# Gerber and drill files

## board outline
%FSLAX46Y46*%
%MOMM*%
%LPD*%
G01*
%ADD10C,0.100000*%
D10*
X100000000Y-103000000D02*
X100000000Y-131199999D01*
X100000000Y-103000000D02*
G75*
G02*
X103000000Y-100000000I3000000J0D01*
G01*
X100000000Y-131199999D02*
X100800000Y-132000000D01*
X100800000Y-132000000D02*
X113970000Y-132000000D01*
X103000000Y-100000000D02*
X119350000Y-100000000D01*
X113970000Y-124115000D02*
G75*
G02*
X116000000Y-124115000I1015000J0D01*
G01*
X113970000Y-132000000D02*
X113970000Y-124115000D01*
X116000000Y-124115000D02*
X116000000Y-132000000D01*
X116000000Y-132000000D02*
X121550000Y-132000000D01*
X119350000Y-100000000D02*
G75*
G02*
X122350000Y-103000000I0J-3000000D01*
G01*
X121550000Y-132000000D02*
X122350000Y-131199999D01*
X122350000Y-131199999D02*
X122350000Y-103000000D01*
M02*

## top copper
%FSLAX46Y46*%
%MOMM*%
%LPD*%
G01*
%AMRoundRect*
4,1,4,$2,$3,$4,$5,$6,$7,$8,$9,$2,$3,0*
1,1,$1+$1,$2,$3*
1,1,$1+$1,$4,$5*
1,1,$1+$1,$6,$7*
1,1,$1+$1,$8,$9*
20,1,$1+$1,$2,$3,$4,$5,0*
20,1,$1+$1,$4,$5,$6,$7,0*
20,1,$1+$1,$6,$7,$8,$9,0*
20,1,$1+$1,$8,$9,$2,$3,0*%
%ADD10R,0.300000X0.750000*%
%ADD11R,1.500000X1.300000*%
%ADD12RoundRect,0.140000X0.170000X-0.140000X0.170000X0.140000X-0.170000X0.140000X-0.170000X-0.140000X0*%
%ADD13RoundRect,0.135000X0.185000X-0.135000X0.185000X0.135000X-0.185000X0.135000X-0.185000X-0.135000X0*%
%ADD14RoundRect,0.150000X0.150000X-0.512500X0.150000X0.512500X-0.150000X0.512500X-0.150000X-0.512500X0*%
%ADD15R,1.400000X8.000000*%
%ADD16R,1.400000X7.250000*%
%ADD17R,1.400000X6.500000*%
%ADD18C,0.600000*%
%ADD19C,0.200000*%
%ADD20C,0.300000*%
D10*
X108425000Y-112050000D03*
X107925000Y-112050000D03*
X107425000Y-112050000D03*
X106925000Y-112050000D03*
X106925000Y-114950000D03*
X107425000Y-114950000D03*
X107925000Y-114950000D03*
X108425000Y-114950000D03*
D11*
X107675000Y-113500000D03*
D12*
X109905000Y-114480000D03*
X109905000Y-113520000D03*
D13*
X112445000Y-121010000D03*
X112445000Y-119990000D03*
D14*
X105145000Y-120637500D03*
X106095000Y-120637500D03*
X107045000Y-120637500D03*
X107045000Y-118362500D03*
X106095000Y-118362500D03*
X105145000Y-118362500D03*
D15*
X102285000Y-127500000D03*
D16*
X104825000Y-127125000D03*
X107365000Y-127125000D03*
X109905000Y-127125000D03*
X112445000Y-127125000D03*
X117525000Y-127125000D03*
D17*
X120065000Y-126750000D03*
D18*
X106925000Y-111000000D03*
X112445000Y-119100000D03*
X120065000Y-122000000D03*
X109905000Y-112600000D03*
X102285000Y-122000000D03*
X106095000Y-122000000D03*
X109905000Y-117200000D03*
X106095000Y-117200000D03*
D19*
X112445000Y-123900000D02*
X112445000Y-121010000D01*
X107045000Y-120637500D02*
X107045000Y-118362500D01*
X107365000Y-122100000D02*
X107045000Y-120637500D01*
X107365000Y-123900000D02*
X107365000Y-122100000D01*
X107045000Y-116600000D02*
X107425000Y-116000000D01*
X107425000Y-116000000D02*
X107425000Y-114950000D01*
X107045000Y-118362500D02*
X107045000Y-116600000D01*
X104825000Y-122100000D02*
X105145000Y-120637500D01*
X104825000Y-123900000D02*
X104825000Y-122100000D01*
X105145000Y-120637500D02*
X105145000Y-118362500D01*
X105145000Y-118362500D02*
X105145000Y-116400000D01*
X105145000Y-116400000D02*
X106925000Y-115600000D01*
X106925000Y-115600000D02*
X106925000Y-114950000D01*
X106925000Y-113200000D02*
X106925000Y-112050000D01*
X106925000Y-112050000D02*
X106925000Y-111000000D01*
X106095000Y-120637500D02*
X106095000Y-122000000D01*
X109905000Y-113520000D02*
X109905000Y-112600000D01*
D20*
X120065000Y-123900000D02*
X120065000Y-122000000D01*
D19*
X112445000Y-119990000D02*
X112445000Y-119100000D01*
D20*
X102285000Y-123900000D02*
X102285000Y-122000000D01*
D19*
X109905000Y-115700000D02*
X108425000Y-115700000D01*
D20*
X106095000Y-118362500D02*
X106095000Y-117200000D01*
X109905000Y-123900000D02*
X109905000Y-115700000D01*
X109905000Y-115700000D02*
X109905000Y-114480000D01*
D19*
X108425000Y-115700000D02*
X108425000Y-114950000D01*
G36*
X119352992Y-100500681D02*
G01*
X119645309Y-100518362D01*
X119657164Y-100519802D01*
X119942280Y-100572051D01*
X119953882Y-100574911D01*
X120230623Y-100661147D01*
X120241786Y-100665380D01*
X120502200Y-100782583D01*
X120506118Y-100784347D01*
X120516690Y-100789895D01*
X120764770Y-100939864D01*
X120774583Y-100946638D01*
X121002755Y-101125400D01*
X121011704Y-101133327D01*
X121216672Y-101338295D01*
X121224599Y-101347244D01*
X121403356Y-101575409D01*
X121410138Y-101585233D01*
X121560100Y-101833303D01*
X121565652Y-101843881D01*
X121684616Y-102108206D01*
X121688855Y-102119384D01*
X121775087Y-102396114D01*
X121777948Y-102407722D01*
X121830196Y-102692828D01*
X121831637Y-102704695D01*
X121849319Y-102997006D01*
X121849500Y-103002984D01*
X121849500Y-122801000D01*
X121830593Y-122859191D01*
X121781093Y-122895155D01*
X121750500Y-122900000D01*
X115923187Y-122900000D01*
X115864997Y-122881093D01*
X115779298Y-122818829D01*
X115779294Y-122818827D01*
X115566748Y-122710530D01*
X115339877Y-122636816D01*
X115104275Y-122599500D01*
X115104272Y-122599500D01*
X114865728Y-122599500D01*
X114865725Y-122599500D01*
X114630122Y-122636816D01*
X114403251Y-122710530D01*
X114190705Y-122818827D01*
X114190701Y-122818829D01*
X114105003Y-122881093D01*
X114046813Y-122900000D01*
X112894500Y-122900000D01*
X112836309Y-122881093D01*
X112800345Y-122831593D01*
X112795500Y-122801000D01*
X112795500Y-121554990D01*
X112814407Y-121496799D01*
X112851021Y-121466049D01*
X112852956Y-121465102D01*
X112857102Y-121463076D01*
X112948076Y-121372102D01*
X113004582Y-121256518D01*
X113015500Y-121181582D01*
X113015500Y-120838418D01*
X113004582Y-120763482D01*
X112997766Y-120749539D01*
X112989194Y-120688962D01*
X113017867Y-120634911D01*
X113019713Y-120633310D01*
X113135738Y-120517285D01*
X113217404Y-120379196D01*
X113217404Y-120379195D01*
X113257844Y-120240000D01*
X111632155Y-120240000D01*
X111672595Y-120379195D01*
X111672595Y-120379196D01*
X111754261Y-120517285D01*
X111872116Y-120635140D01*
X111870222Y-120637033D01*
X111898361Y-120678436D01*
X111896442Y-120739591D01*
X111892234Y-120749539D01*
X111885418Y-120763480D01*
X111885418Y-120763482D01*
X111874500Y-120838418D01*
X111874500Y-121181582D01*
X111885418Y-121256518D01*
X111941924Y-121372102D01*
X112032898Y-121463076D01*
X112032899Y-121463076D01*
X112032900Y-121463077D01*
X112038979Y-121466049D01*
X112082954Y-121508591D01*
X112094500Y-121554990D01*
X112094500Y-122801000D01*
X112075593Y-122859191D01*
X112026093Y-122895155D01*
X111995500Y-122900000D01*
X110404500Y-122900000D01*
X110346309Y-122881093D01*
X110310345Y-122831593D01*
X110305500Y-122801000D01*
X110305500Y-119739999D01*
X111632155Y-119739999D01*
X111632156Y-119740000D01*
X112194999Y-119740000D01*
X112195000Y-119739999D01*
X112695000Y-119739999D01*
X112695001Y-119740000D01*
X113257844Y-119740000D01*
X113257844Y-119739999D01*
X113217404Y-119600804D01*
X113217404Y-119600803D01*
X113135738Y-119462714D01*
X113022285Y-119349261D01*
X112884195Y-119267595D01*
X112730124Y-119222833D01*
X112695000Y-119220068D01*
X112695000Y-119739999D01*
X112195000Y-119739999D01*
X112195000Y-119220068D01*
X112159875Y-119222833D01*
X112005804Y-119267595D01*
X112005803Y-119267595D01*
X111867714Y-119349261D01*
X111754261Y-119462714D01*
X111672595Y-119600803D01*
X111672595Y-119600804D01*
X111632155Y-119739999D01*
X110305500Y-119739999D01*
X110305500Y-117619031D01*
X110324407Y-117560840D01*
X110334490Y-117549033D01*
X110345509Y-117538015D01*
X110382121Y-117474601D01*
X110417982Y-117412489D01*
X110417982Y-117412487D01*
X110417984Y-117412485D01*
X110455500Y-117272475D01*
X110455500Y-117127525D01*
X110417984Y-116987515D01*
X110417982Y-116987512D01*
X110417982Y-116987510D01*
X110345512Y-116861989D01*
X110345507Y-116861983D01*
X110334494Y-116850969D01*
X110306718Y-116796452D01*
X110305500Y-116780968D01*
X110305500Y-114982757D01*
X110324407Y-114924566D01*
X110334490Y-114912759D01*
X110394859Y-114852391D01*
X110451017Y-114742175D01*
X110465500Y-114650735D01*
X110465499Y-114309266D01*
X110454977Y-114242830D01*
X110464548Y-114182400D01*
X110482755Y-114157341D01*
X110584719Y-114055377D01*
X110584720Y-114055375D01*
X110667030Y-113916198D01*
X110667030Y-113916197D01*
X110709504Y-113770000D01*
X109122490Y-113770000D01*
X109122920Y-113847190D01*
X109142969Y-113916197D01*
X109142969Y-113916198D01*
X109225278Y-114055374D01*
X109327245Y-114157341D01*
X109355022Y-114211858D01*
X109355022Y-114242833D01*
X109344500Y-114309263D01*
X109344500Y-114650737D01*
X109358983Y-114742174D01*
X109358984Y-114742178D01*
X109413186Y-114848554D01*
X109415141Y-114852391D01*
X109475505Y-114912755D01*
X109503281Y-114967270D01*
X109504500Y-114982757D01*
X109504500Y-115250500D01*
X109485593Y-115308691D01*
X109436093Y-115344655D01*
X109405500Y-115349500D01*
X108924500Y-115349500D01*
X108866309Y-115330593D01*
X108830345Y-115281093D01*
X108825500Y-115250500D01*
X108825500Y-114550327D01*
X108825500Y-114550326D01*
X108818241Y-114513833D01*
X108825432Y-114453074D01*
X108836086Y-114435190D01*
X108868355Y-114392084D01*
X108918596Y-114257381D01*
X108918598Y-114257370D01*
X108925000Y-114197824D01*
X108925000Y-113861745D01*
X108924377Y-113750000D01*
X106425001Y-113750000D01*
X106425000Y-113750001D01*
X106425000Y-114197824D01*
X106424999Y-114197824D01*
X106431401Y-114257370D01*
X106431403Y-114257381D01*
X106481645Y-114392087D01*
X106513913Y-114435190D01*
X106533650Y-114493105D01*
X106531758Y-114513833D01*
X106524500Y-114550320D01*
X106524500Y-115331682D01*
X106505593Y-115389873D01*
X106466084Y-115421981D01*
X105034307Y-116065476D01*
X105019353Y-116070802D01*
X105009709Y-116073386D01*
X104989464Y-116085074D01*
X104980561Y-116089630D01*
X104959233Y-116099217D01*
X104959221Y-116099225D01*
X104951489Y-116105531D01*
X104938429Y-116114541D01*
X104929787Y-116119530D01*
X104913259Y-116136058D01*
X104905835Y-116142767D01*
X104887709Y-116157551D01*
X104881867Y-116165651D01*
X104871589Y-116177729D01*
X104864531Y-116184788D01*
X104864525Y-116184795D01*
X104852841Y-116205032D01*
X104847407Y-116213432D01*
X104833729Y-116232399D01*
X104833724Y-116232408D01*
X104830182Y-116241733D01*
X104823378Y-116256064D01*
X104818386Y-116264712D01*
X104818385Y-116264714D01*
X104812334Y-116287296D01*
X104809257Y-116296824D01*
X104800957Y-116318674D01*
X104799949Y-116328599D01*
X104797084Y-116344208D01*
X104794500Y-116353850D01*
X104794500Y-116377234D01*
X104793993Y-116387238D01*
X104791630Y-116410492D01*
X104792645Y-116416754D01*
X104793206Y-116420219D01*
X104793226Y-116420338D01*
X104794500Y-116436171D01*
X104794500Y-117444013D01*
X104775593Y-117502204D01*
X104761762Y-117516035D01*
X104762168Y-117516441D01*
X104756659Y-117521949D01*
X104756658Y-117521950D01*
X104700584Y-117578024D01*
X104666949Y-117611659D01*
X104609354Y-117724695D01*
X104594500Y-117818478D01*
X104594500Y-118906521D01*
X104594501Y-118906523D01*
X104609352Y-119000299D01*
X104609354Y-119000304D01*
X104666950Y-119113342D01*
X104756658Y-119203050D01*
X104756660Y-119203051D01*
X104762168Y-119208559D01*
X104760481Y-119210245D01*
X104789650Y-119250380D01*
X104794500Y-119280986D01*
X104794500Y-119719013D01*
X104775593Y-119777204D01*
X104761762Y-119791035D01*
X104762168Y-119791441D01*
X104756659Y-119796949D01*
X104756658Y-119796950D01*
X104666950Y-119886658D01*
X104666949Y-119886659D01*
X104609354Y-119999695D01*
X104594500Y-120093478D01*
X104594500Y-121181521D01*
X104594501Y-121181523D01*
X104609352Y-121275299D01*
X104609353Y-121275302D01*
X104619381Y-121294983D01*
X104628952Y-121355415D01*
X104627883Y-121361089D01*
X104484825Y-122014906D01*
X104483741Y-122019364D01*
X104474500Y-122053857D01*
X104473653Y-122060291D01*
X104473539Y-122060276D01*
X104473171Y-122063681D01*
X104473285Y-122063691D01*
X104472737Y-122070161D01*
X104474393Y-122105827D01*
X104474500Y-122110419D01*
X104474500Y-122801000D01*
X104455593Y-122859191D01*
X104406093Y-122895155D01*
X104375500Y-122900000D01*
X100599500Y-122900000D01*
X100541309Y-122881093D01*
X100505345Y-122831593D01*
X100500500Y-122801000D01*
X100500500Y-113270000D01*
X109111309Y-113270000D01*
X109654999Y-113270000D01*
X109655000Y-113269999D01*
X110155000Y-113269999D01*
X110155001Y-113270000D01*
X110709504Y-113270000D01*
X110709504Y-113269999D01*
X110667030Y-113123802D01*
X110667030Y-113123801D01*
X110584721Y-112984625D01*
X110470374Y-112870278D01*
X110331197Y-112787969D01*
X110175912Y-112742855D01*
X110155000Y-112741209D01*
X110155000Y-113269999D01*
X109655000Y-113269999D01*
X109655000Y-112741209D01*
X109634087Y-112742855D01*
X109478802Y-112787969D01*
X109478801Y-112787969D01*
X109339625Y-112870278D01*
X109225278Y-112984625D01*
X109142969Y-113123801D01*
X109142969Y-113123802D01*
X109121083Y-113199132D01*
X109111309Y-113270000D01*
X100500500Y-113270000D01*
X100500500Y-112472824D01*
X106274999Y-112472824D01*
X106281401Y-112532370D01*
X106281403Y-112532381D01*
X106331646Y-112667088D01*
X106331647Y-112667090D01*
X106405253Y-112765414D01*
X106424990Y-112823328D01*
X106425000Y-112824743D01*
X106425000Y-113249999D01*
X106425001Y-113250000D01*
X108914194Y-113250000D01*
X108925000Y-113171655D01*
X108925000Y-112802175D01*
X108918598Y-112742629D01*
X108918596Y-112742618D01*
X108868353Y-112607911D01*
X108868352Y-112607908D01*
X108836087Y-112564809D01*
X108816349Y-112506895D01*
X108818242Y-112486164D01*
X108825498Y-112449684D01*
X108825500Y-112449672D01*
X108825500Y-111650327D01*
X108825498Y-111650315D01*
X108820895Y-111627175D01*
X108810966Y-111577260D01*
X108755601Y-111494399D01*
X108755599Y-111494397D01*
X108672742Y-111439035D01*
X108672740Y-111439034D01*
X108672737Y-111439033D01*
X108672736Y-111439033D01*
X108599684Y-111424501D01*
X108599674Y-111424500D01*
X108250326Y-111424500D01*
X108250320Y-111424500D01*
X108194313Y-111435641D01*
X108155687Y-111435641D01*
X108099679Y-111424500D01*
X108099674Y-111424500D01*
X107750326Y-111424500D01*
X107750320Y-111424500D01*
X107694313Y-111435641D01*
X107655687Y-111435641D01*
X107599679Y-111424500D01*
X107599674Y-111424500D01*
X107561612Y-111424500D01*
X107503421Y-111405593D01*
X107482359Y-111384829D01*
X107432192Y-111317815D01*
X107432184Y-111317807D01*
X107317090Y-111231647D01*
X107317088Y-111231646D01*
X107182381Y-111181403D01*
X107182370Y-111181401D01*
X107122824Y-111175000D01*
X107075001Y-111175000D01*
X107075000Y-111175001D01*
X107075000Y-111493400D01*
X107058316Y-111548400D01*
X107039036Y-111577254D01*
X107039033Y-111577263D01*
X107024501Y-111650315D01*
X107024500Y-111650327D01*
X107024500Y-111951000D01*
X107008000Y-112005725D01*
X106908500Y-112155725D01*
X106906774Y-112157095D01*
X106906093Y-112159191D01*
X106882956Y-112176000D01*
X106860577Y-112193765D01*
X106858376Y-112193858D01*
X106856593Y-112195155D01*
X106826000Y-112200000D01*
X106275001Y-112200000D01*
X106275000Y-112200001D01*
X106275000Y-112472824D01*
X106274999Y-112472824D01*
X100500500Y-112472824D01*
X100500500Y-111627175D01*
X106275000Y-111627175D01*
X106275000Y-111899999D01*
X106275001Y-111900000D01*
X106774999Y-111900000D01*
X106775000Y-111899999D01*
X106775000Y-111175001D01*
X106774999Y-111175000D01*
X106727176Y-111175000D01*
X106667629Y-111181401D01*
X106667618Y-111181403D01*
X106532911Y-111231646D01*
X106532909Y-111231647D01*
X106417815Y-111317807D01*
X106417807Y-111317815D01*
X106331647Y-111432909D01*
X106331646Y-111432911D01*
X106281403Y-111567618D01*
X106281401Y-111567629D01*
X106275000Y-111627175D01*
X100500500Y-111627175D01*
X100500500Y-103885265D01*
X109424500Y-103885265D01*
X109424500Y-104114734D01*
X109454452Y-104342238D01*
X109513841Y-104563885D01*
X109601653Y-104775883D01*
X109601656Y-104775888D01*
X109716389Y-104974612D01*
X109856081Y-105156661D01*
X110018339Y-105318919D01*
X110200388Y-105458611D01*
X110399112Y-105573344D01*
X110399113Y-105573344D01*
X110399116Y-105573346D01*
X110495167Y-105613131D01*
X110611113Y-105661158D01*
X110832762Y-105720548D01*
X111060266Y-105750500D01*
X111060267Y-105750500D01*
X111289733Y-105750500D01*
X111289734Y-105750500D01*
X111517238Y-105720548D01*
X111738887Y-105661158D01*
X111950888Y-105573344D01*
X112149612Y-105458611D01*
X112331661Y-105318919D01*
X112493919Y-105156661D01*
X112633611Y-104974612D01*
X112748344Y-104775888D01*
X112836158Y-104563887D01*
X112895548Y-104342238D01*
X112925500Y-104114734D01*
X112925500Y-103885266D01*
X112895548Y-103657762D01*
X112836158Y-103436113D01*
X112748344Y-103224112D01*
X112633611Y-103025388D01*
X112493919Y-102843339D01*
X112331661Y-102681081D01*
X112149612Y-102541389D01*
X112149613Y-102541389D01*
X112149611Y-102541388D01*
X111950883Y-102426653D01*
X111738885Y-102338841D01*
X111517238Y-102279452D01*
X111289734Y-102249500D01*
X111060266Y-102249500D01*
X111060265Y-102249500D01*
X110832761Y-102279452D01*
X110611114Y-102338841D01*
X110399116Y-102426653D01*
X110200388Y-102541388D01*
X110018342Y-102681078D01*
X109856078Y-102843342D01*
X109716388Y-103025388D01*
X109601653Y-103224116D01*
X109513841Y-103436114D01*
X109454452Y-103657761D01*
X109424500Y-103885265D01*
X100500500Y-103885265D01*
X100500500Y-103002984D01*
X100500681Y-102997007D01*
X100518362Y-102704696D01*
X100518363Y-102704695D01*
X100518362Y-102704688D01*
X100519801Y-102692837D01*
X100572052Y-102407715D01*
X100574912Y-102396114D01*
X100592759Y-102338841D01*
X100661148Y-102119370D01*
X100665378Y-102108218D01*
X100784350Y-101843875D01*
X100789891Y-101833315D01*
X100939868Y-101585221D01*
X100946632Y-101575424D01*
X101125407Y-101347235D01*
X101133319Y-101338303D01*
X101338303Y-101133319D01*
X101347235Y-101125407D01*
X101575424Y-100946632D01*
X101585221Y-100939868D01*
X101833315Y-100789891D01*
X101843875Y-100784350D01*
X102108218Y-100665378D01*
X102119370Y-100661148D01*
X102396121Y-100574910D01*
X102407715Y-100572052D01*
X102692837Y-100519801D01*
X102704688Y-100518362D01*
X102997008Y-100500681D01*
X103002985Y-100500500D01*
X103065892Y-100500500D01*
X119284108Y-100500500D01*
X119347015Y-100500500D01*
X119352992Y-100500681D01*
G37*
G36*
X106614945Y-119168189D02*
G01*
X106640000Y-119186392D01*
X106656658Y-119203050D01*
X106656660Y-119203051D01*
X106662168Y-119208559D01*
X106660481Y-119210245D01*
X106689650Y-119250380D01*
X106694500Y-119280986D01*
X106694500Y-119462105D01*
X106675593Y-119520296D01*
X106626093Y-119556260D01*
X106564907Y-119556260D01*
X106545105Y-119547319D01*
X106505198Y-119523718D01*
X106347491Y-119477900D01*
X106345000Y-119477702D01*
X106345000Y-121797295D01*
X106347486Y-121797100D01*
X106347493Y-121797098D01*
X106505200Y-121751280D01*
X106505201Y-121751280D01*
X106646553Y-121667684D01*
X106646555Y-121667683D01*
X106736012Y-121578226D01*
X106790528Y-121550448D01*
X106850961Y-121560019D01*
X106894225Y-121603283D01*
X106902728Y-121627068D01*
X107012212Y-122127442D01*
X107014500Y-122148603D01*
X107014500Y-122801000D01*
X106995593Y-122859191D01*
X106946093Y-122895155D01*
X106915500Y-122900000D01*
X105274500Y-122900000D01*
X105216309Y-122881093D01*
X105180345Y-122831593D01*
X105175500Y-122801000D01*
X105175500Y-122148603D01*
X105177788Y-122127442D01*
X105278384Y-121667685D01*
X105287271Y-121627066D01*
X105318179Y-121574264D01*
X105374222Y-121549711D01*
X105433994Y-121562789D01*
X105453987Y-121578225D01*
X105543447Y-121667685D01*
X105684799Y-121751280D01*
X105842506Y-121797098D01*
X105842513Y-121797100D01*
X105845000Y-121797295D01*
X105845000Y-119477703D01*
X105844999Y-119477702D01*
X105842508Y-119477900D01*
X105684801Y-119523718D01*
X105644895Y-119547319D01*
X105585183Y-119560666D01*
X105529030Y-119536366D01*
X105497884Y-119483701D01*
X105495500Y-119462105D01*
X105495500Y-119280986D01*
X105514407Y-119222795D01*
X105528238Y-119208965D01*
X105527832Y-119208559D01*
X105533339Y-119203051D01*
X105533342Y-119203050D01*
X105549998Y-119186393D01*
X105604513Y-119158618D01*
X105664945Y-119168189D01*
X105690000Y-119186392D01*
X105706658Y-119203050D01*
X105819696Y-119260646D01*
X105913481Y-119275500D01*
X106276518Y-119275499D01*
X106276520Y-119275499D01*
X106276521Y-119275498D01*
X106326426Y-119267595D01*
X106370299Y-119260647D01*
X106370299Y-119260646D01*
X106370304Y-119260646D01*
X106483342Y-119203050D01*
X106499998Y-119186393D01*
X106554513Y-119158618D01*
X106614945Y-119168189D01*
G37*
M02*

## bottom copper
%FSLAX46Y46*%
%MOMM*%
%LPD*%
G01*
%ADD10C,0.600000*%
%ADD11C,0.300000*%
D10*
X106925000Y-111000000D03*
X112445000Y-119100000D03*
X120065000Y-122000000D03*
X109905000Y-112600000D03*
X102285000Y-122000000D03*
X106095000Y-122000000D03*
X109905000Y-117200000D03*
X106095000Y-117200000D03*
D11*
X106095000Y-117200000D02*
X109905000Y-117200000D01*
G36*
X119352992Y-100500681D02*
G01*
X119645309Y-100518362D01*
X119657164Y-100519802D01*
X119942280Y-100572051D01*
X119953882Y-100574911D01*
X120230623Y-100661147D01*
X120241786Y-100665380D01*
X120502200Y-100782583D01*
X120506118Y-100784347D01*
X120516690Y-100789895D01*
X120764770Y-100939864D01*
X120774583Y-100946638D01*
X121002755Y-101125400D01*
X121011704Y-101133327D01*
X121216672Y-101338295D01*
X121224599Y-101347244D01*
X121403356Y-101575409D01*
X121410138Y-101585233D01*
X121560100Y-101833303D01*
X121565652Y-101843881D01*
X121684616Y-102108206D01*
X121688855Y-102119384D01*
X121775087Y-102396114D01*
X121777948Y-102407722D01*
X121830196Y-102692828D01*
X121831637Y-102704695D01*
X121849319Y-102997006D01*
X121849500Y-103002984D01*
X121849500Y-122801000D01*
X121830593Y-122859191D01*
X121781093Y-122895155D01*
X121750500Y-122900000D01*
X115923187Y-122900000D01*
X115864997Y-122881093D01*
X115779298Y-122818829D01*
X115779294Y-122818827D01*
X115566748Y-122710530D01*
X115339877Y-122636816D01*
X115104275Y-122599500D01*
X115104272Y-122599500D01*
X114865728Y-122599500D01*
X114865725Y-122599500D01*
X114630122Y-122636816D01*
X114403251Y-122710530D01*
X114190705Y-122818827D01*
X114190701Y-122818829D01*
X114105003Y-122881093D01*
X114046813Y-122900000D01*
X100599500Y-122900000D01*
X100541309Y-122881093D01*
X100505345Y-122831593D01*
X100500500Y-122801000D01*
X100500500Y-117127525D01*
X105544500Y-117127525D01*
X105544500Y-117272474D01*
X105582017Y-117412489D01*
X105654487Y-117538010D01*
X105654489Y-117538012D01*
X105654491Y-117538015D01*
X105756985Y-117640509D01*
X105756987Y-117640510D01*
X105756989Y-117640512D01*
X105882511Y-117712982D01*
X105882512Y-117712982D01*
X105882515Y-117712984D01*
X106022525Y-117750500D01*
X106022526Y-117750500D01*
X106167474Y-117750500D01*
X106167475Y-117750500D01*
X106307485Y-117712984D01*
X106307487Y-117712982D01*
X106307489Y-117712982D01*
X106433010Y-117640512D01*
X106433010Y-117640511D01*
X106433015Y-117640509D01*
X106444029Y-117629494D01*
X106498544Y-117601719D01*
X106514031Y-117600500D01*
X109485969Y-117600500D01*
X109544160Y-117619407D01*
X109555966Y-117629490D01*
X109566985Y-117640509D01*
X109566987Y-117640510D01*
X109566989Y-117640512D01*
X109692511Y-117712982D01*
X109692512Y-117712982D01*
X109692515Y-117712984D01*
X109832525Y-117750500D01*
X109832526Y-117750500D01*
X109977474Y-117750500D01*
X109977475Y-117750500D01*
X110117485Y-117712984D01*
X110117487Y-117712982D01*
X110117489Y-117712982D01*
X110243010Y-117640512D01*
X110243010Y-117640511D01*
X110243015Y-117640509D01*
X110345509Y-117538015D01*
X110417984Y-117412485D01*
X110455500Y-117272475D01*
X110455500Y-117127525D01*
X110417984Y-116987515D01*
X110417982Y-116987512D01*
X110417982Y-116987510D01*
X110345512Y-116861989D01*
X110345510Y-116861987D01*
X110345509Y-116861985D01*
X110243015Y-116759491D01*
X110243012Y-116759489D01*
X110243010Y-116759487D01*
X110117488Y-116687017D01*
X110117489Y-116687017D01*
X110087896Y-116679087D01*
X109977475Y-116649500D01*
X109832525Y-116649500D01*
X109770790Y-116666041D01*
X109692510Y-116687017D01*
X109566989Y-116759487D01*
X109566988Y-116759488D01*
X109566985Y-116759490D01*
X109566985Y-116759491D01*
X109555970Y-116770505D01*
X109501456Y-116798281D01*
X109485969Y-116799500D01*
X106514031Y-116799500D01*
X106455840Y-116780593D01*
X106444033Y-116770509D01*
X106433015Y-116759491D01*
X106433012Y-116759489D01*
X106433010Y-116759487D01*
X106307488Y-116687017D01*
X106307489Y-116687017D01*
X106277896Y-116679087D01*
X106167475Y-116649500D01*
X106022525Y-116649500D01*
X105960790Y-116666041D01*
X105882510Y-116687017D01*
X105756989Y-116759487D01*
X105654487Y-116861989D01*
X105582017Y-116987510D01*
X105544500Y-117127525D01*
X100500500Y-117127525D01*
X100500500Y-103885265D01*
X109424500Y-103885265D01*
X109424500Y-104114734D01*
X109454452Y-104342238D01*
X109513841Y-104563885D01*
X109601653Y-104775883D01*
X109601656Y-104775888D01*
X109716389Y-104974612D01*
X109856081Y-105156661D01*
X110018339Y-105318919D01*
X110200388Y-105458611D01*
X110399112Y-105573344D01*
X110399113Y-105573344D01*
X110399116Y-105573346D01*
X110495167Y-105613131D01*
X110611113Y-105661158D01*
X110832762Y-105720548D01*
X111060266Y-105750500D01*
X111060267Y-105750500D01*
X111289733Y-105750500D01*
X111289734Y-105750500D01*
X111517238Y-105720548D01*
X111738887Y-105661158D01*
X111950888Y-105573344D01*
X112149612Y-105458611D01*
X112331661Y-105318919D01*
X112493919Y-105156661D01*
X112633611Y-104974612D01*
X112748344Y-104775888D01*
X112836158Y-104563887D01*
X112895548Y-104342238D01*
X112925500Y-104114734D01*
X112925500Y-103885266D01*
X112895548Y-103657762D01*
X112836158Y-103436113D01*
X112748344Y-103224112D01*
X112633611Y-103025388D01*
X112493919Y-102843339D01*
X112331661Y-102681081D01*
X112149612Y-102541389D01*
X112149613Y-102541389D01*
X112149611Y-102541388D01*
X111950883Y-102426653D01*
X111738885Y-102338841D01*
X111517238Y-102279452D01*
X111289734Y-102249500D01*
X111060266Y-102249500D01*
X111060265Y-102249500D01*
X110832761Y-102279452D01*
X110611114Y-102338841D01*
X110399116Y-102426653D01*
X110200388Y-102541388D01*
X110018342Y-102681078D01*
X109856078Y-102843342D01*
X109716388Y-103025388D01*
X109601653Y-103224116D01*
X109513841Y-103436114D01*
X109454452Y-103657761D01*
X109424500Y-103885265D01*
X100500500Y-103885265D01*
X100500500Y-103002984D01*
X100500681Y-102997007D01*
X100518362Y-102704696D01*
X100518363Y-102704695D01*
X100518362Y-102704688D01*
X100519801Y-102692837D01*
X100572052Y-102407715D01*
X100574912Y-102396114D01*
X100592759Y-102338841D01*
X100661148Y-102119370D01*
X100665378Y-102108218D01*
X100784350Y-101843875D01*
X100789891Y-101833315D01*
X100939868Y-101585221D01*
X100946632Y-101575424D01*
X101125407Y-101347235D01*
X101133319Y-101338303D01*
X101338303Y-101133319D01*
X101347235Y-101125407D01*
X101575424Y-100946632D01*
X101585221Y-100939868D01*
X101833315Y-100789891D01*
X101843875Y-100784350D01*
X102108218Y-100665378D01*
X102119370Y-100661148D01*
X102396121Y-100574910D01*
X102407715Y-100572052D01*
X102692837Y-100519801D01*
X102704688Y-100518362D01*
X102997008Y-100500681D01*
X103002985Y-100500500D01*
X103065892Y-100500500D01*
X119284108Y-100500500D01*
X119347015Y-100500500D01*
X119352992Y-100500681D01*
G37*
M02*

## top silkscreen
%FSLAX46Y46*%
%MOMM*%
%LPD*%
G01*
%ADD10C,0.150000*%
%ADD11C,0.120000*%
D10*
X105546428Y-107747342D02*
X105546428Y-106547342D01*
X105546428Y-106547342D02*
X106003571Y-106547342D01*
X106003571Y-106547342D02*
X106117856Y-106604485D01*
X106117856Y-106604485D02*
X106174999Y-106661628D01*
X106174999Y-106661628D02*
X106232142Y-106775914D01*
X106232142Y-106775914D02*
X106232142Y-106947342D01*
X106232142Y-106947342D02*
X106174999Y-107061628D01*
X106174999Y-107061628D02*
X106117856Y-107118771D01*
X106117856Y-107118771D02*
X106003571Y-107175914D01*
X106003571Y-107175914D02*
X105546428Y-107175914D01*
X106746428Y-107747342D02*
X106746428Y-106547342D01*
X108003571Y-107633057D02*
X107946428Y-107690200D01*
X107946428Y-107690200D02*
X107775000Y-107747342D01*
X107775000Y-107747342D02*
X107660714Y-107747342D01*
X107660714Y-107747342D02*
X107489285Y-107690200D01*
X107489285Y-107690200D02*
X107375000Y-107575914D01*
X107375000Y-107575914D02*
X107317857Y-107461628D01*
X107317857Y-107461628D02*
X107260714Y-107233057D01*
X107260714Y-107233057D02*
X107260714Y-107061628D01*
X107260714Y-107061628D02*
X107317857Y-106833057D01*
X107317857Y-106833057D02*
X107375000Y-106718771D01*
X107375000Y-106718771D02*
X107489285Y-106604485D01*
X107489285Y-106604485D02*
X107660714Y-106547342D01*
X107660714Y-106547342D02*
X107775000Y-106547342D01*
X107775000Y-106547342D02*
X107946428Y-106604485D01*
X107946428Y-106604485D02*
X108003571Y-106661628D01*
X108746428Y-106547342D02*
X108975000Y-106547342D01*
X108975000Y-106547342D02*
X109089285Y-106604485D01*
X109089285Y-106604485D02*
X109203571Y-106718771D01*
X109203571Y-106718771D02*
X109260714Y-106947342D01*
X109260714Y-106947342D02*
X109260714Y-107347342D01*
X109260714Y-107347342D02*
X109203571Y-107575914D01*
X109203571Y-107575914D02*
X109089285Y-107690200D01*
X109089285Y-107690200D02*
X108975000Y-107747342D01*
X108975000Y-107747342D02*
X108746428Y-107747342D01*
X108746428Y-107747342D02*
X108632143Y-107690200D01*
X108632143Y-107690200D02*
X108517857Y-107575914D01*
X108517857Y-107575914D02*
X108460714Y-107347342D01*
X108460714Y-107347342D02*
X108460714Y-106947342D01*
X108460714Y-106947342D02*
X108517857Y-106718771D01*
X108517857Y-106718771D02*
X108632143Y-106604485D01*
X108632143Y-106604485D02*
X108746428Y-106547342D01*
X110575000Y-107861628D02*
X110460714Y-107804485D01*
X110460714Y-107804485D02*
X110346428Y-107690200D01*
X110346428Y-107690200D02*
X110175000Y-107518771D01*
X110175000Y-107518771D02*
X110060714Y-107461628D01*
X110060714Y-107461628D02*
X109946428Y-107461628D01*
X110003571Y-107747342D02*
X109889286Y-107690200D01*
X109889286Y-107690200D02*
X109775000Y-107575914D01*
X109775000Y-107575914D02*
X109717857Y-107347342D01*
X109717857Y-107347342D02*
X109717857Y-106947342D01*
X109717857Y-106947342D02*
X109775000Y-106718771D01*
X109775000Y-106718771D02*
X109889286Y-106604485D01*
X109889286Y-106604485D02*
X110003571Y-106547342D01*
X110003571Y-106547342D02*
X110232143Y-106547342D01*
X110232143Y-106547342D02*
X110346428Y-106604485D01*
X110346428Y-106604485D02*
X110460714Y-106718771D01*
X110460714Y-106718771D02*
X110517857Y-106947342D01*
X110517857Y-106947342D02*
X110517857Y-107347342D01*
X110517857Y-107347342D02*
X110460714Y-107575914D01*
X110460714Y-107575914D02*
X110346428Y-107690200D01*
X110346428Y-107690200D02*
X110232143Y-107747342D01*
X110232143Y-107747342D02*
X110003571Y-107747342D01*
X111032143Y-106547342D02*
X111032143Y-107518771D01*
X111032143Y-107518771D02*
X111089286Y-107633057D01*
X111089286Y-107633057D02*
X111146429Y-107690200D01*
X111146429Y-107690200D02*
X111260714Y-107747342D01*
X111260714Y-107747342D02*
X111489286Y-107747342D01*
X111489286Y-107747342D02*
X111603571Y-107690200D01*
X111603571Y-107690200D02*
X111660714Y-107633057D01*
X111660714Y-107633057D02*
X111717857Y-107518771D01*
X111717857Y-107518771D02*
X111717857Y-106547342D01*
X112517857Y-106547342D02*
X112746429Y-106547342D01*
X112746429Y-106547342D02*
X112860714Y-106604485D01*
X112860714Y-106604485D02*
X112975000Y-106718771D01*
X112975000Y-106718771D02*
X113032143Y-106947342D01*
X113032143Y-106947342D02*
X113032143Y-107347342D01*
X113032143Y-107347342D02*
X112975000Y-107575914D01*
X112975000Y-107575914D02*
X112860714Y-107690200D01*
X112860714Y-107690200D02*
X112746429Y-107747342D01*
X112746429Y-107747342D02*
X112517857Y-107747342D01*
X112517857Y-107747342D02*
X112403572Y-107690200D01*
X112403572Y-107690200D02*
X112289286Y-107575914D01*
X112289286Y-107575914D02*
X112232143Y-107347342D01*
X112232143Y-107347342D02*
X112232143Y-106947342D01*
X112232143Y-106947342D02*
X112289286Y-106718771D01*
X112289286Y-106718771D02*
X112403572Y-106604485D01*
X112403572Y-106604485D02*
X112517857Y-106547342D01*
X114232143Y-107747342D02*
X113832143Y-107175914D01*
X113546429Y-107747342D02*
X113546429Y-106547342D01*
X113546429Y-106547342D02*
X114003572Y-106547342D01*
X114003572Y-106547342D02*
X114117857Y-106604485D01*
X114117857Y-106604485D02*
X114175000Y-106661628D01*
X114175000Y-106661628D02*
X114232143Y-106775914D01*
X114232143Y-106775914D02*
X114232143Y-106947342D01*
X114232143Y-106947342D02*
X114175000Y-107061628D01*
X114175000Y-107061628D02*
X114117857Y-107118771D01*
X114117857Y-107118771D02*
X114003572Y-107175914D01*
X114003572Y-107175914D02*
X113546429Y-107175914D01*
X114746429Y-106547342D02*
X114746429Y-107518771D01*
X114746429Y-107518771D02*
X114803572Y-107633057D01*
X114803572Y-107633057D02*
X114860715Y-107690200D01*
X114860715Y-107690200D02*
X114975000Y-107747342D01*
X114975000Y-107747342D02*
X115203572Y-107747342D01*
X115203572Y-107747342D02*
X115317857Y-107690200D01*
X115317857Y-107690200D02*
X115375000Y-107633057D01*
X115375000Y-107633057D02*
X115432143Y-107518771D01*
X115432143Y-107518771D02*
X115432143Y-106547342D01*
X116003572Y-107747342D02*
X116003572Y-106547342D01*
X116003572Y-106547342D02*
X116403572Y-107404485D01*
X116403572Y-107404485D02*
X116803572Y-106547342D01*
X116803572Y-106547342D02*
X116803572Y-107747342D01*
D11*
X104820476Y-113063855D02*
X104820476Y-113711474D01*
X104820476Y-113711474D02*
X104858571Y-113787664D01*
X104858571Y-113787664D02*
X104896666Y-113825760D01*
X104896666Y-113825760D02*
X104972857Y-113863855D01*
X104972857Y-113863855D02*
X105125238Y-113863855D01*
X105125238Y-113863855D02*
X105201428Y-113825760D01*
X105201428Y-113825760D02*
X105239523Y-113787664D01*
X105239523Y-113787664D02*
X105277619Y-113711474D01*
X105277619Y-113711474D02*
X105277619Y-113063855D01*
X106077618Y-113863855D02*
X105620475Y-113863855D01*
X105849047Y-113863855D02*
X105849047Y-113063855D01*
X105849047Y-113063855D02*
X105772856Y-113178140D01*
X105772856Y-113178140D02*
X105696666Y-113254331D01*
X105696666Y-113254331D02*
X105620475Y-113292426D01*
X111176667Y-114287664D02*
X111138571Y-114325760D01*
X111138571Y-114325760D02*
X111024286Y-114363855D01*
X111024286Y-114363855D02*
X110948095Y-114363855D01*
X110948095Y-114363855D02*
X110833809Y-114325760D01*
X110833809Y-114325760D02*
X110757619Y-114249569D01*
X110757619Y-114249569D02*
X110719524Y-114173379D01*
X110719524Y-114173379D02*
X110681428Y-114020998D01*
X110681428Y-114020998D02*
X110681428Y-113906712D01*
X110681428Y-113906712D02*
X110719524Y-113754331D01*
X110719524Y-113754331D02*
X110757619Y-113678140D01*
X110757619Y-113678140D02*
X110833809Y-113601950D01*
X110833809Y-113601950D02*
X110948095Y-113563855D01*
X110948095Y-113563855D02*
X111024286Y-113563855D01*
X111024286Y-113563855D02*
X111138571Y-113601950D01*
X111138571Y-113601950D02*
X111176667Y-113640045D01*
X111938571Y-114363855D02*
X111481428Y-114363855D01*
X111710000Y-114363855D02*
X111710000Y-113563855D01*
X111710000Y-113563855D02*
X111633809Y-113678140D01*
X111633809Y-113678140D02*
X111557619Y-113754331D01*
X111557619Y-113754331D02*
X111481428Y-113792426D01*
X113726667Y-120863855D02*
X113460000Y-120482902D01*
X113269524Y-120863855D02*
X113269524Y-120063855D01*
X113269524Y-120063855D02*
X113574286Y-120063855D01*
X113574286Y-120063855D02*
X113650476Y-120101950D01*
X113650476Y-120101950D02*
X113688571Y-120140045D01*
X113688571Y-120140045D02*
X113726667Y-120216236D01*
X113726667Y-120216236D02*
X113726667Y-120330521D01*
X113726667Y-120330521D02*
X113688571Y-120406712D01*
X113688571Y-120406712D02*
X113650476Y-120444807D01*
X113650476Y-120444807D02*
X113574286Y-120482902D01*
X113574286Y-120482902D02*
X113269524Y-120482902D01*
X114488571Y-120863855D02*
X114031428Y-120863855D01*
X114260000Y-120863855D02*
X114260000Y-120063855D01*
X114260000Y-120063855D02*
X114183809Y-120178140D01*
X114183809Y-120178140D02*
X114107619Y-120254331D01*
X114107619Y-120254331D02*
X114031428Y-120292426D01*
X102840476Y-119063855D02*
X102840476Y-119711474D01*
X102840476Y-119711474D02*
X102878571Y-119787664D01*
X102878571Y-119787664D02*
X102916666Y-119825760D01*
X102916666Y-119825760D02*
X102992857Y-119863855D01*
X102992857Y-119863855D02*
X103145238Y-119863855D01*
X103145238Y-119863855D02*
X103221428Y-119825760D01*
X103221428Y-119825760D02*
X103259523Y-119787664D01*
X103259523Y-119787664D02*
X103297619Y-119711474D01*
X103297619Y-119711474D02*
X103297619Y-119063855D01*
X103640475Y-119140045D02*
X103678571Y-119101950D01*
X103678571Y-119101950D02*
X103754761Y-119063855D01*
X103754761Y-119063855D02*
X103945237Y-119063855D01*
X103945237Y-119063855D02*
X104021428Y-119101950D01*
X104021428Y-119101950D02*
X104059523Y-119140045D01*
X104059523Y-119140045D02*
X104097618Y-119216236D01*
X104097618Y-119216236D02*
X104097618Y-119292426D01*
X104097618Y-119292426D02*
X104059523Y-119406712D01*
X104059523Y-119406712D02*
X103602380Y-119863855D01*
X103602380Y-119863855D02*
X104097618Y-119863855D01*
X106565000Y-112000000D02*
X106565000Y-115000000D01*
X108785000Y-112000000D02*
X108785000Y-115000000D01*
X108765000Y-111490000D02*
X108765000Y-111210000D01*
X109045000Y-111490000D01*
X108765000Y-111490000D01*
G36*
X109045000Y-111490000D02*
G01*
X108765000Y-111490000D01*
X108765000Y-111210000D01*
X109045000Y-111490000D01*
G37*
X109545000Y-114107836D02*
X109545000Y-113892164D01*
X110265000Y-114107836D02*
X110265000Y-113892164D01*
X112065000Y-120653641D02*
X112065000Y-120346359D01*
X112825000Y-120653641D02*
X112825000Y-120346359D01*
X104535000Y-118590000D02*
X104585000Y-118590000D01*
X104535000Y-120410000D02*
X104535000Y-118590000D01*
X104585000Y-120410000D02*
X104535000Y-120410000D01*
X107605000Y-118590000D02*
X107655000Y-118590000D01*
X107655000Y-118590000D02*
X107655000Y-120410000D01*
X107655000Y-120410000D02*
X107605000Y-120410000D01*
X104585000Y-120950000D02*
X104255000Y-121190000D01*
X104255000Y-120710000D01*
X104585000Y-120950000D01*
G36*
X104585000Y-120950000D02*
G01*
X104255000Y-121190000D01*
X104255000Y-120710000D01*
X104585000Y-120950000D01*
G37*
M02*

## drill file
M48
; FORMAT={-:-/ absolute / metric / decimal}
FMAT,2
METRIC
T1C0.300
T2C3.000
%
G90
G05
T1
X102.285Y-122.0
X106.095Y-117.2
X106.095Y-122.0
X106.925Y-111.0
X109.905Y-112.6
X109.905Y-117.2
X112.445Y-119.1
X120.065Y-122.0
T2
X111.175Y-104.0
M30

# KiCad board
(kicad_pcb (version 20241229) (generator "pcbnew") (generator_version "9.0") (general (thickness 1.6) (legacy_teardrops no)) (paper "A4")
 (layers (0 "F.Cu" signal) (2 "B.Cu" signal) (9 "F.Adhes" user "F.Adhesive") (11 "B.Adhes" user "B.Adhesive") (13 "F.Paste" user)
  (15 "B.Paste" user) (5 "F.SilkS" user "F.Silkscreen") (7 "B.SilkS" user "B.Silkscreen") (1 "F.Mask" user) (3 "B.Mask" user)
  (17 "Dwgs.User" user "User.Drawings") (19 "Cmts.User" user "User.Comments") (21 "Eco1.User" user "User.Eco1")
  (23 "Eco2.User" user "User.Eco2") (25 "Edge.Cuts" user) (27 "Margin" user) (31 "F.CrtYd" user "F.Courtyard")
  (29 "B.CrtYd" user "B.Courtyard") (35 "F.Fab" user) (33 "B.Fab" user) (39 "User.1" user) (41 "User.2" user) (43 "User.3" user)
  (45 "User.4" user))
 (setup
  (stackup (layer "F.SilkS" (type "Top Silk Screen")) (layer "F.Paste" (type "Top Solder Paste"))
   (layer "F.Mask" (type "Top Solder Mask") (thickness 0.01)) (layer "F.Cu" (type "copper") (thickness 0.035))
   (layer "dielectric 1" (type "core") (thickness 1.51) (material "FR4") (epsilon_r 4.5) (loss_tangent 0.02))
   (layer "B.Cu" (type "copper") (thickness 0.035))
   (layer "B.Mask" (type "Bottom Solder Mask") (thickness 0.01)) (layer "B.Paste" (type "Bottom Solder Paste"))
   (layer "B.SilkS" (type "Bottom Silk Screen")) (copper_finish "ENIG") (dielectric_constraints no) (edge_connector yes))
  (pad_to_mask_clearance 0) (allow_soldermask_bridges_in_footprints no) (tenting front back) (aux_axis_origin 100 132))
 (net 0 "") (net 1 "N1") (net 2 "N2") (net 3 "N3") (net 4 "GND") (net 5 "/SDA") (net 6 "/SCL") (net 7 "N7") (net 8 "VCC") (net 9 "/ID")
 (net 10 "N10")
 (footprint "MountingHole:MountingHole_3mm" (layer "F.Cu") (at 111.175 104)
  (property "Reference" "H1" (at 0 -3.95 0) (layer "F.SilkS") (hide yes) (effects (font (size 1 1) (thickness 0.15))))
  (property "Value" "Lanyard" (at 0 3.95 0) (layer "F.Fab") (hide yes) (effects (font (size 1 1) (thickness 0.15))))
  (pad "" np_thru_hole circle (at 0 0) (size 3 3) (drill 3) (layers "*.Cu" "*.Mask")))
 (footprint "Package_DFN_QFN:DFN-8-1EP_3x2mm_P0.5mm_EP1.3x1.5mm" (layer "F.Cu") (at 107.675 113.5 -90)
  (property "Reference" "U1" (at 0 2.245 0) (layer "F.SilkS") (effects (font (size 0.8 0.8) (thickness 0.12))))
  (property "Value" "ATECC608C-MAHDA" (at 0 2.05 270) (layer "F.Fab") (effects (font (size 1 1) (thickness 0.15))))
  (fp_line (start -1.5 1.11) (end 1.5 1.11) (stroke (width 0.12) (type solid)) (layer "F.SilkS"))
  (fp_line (start -1.5 -1.11) (end 1.5 -1.11) (stroke (width 0.12) (type solid)) (layer "F.SilkS"))
  (fp_poly
   (pts (xy -2.01 -1.09) (xy -2.29 -1.09) (xy -2.01 -1.37) (xy -2.01 -1.09)) (stroke (width 0.12) (type solid)) (fill yes) (layer "F.SilkS"))
  (pad "" smd rect (at -0.325 -0.375 270) (size 0.5 0.6) (layers "F.Paste"))
  (pad "" smd rect (at -0.325 0.375 270) (size 0.5 0.6) (layers "F.Paste"))
  (pad "" smd rect (at 0.325 -0.375 270) (size 0.5 0.6) (layers "F.Paste"))
  (pad "" smd rect (at 0.325 0.375 270) (size 0.5 0.6) (layers "F.Paste"))
  (pad "1" smd rect (at -1.45 -0.75 270) (size 0.75 0.3) (layers "F.Cu" "F.Mask" "F.Paste") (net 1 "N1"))
  (pad "2" smd rect (at -1.45 -0.25 270) (size 0.75 0.3) (layers "F.Cu" "F.Mask" "F.Paste") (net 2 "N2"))
  (pad "3" smd rect (at -1.45 0.25 270) (size 0.75 0.3) (layers "F.Cu" "F.Mask" "F.Paste") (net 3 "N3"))
  (pad "4" smd rect (at -1.45 0.75 270) (size 0.75 0.3) (layers "F.Cu" "F.Mask" "F.Paste") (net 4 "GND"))
  (pad "5" smd rect (at 1.45 0.75 270) (size 0.75 0.3) (layers "F.Cu" "F.Mask" "F.Paste") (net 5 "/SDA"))
  (pad "6" smd rect (at 1.45 0.25 270) (size 0.75 0.3) (layers "F.Cu" "F.Mask" "F.Paste") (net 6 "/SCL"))
  (pad "7" smd rect (at 1.45 -0.25 270) (size 0.75 0.3) (layers "F.Cu" "F.Mask" "F.Paste") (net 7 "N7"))
  (pad "8" smd rect (at 1.45 -0.75 270) (size 0.75 0.3) (layers "F.Cu" "F.Mask" "F.Paste") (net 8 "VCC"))
  (pad "9" smd rect (at 0 0 270) (size 1.3 1.5) (layers "F.Cu" "F.Mask") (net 4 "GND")))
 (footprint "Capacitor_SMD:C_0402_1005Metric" (layer "F.Cu") (at 109.905 114 90)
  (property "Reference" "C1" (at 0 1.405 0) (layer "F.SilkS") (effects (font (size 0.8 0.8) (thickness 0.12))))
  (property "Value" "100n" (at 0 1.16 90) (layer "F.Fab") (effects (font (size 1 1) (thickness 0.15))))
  (fp_line (start -0.107836 -0.36) (end 0.107836 -0.36) (stroke (width 0.12) (type solid)) (layer "F.SilkS"))
  (fp_line (start -0.107836 0.36) (end 0.107836 0.36) (stroke (width 0.12) (type solid)) (layer "F.SilkS"))
  (pad "1" smd roundrect (at -0.48 0 90) (size 0.56 0.62) (layers "F.Cu" "F.Mask" "F.Paste") (roundrect_rratio 0.25) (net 8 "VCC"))
  (pad "2" smd roundrect (at 0.48 0 90) (size 0.56 0.62) (layers "F.Cu" "F.Mask" "F.Paste") (roundrect_rratio 0.25) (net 4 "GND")))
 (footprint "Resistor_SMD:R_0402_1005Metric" (layer "F.Cu") (at 112.445 120.5 90)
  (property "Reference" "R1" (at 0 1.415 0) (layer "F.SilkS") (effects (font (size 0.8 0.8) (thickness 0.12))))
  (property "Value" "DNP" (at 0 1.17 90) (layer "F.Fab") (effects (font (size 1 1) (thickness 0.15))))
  (fp_line (start -0.153641 -0.38) (end 0.153641 -0.38) (stroke (width 0.12) (type solid)) (layer "F.SilkS"))
  (fp_line (start -0.153641 0.38) (end 0.153641 0.38) (stroke (width 0.12) (type solid)) (layer "F.SilkS"))
  (pad "1" smd roundrect (at -0.51 0 90) (size 0.54 0.64) (layers "F.Cu" "F.Mask" "F.Paste") (roundrect_rratio 0.25) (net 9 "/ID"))
  (pad "2" smd roundrect (at 0.51 0 90) (size 0.54 0.64) (layers "F.Cu" "F.Mask" "F.Paste") (roundrect_rratio 0.25) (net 4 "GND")))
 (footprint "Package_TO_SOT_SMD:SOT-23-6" (layer "F.Cu") (at 106.095 119.5 90)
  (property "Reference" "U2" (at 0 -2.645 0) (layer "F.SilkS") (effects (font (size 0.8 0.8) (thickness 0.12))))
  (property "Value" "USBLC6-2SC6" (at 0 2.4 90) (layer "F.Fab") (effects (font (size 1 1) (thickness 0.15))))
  (fp_line (start 0.91 -1.56) (end 0.91 -1.51) (stroke (width 0.12) (type solid)) (layer "F.SilkS"))
  (fp_line (start -0.91 -1.56) (end 0.91 -1.56) (stroke (width 0.12) (type solid)) (layer "F.SilkS"))
  (fp_line (start -0.91 -1.51) (end -0.91 -1.56) (stroke (width 0.12) (type solid)) (layer "F.SilkS"))
  (fp_line (start 0.91 1.51) (end 0.91 1.56) (stroke (width 0.12) (type solid)) (layer "F.SilkS"))
  (fp_line (start 0.91 1.56) (end -0.91 1.56) (stroke (width 0.12) (type solid)) (layer "F.SilkS"))
  (fp_line (start -0.91 1.56) (end -0.91 1.51) (stroke (width 0.12) (type solid)) (layer "F.SilkS"))
  (fp_poly (pts (xy -1.45 -1.51) (xy -1.69 -1.84) (xy -1.21 -1.84)) (stroke (width 0.12) (type solid)) (fill yes) (layer "F.SilkS"))
  (pad "1" smd roundrect (at -1.1375 -0.95 90) (size 1.325 0.6) (layers "F.Cu" "F.Mask" "F.Paste") (roundrect_rratio 0.25) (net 5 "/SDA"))
  (pad "2" smd roundrect (at -1.1375 0 90) (size 1.325 0.6) (layers "F.Cu" "F.Mask" "F.Paste") (roundrect_rratio 0.25) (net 4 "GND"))
  (pad "3" smd roundrect (at -1.1375 0.95 90) (size 1.325 0.6) (layers "F.Cu" "F.Mask" "F.Paste") (roundrect_rratio 0.25) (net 6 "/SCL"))
  (pad "4" smd roundrect (at 1.1375 0.95 90) (size 1.325 0.6) (layers "F.Cu" "F.Mask" "F.Paste") (roundrect_rratio 0.25) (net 6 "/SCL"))
  (pad "5" smd roundrect (at 1.1375 0 90) (size 1.325 0.6) (layers "F.Cu" "F.Mask" "F.Paste") (roundrect_rratio 0.25) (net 8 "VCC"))
  (pad "6" smd roundrect (at 1.1375 -0.95 90) (size 1.325 0.6) (layers "F.Cu" "F.Mask" "F.Paste") (roundrect_rratio 0.25) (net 5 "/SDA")))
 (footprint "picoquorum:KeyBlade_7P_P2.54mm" (layer "F.Cu") (at 111.175 132)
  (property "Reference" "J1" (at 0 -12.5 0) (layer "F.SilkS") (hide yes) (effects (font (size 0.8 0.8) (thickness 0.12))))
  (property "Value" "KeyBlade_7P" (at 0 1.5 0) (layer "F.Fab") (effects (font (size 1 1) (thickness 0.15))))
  (pad "1" smd rect (at -8.89 -4.5) (size 1.4 8) (layers "F.Cu" "F.Mask") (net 4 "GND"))
  (pad "2" smd rect (at -6.35 -4.875) (size 1.4 7.25) (layers "F.Cu" "F.Mask") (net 5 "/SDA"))
  (pad "3" smd rect (at -3.81 -4.875) (size 1.4 7.25) (layers "F.Cu" "F.Mask") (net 6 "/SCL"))
  (pad "4" smd rect (at -1.27 -4.875) (size 1.4 7.25) (layers "F.Cu" "F.Mask") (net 8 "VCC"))
  (pad "5" smd rect (at 1.27 -4.875) (size 1.4 7.25) (layers "F.Cu" "F.Mask") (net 9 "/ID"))
  (pad "7" smd rect (at 6.35 -4.875) (size 1.4 7.25) (layers "F.Cu" "F.Mask") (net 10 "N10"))
  (pad "8" smd rect (at 8.89 -5.25) (size 1.4 6.5) (layers "F.Cu" "F.Mask") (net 4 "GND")))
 (gr_line (start 100 103) (end 100 131.199999) (stroke (width 0.1) (type default)) (layer "Edge.Cuts"))
 (gr_arc (start 100 103) (mid 100.87868 100.87868) (end 103 100) (stroke (width 0.1) (type default)) (layer "Edge.Cuts"))
 (gr_line (start 100 131.199999) (end 100.8 132) (stroke (width 0.1) (type default)) (layer "Edge.Cuts"))
 (gr_line (start 100.8 132) (end 113.97 132) (stroke (width 0.1) (type default)) (layer "Edge.Cuts"))
 (gr_line (start 103 100) (end 119.35 100) (stroke (width 0.1) (type default)) (layer "Edge.Cuts"))
 (gr_arc (start 113.97 124.115) (mid 114.985 123.1) (end 116 124.115) (stroke (width 0.1) (type default)) (layer "Edge.Cuts"))
 (gr_line (start 113.97 132) (end 113.97 124.115) (stroke (width 0.1) (type default)) (layer "Edge.Cuts"))
 (gr_line (start 116 124.115) (end 116 132) (stroke (width 0.1) (type default)) (layer "Edge.Cuts"))
 (gr_line (start 116 132) (end 121.55 132) (stroke (width 0.1) (type default)) (layer "Edge.Cuts"))
 (gr_arc (start 119.35 100) (mid 121.47132 100.87868) (end 122.35 103) (stroke (width 0.1) (type default)) (layer "Edge.Cuts"))
 (gr_line (start 121.55 132) (end 122.35 131.199999) (stroke (width 0.1) (type default)) (layer "Edge.Cuts"))
 (gr_line (start 122.35 131.199999) (end 122.35 103) (stroke (width 0.1) (type default)) (layer "Edge.Cuts"))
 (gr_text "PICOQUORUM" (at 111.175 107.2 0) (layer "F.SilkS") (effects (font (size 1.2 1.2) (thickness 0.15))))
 (segment (start 112.445 123.9) (end 112.445 121.01) (width 0.2) (layer "F.Cu") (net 9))
 (segment (start 107.045 120.6375) (end 107.045 118.3625) (width 0.2) (layer "F.Cu") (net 6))
 (segment (start 107.365 122.1) (end 107.045 120.6375) (width 0.2) (layer "F.Cu") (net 6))
 (segment (start 107.365 123.9) (end 107.365 122.1) (width 0.2) (layer "F.Cu") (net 6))
 (segment (start 107.045 116.6) (end 107.425 116) (width 0.2) (layer "F.Cu") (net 6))
 (segment (start 107.425 116) (end 107.425 114.95) (width 0.2) (layer "F.Cu") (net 6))
 (segment (start 107.045 118.3625) (end 107.045 116.6) (width 0.2) (layer "F.Cu") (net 6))
 (segment (start 104.825 122.1) (end 105.145 120.6375) (width 0.2) (layer "F.Cu") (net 5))
 (segment (start 104.825 123.9) (end 104.825 122.1) (width 0.2) (layer "F.Cu") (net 5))
 (segment (start 105.145 120.6375) (end 105.145 118.3625) (width 0.2) (layer "F.Cu") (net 5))
 (segment (start 105.145 118.3625) (end 105.145 116.4) (width 0.2) (layer "F.Cu") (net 5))
 (segment (start 105.145 116.4) (end 106.925 115.6) (width 0.2) (layer "F.Cu") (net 5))
 (segment (start 106.925 115.6) (end 106.925 114.95) (width 0.2) (layer "F.Cu") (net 5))
 (segment (start 106.925 113.2) (end 106.925 112.05) (width 0.2) (layer "F.Cu") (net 4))
 (segment (start 106.925 112.05) (end 106.925 111) (width 0.2) (layer "F.Cu") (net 4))
 (segment (start 106.095 120.6375) (end 106.095 122) (width 0.2) (layer "F.Cu") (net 4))
 (segment (start 109.905 113.52) (end 109.905 112.6) (width 0.2) (layer "F.Cu") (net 4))
 (segment (start 120.065 123.9) (end 120.065 122) (width 0.3) (layer "F.Cu") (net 4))
 (segment (start 112.445 119.99) (end 112.445 119.1) (width 0.2) (layer "F.Cu") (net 4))
 (segment (start 102.285 123.9) (end 102.285 122) (width 0.3) (layer "F.Cu") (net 4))
 (via (at 106.925 111) (size 0.6) (drill 0.3) (layers "F.Cu" "B.Cu") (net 4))
 (via (at 112.445 119.1) (size 0.6) (drill 0.3) (layers "F.Cu" "B.Cu") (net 4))
 (via (at 120.065 122) (size 0.6) (drill 0.3) (layers "F.Cu" "B.Cu") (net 4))
 (via (at 109.905 112.6) (size 0.6) (drill 0.3) (layers "F.Cu" "B.Cu") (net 4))
 (via (at 102.285 122) (size 0.6) (drill 0.3) (layers "F.Cu" "B.Cu") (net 4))
 (via (at 106.095 122) (size 0.6) (drill 0.3) (layers "F.Cu" "B.Cu") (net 4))
 (segment (start 109.905 115.7) (end 108.425 115.7) (width 0.2) (layer "F.Cu") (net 8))
 (segment (start 106.095 118.3625) (end 106.095 117.2) (width 0.3) (layer "F.Cu") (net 8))
 (segment (start 109.905 123.9) (end 109.905 115.7) (width 0.3) (layer "F.Cu") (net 8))
 (segment (start 109.905 115.7) (end 109.905 114.48) (width 0.3) (layer "F.Cu") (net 8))
 (segment (start 108.425 115.7) (end 108.425 114.95) (width 0.2) (layer "F.Cu") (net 8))
 (via (at 109.905 117.2) (size 0.6) (drill 0.3) (layers "F.Cu" "B.Cu") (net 8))
 (via (at 106.095 117.2) (size 0.6) (drill 0.3) (layers "F.Cu" "B.Cu") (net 8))
 (segment (start 106.095 117.2) (end 109.905 117.2) (width 0.3) (layer "B.Cu") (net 8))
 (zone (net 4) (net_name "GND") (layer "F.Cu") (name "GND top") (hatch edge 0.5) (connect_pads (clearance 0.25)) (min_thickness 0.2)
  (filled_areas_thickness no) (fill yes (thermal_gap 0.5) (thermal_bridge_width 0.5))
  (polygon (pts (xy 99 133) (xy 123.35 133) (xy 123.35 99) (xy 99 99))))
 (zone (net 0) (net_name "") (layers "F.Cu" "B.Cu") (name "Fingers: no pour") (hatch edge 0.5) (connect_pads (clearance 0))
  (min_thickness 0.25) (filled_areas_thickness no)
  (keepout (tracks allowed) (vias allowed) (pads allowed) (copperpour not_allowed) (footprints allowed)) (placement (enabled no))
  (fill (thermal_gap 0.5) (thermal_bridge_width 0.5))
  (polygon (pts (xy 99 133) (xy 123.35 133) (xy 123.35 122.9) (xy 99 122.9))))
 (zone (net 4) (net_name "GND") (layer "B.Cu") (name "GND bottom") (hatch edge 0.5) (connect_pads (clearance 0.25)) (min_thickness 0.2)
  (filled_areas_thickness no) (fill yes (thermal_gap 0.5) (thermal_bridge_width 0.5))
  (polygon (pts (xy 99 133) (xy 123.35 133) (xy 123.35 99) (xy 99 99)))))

